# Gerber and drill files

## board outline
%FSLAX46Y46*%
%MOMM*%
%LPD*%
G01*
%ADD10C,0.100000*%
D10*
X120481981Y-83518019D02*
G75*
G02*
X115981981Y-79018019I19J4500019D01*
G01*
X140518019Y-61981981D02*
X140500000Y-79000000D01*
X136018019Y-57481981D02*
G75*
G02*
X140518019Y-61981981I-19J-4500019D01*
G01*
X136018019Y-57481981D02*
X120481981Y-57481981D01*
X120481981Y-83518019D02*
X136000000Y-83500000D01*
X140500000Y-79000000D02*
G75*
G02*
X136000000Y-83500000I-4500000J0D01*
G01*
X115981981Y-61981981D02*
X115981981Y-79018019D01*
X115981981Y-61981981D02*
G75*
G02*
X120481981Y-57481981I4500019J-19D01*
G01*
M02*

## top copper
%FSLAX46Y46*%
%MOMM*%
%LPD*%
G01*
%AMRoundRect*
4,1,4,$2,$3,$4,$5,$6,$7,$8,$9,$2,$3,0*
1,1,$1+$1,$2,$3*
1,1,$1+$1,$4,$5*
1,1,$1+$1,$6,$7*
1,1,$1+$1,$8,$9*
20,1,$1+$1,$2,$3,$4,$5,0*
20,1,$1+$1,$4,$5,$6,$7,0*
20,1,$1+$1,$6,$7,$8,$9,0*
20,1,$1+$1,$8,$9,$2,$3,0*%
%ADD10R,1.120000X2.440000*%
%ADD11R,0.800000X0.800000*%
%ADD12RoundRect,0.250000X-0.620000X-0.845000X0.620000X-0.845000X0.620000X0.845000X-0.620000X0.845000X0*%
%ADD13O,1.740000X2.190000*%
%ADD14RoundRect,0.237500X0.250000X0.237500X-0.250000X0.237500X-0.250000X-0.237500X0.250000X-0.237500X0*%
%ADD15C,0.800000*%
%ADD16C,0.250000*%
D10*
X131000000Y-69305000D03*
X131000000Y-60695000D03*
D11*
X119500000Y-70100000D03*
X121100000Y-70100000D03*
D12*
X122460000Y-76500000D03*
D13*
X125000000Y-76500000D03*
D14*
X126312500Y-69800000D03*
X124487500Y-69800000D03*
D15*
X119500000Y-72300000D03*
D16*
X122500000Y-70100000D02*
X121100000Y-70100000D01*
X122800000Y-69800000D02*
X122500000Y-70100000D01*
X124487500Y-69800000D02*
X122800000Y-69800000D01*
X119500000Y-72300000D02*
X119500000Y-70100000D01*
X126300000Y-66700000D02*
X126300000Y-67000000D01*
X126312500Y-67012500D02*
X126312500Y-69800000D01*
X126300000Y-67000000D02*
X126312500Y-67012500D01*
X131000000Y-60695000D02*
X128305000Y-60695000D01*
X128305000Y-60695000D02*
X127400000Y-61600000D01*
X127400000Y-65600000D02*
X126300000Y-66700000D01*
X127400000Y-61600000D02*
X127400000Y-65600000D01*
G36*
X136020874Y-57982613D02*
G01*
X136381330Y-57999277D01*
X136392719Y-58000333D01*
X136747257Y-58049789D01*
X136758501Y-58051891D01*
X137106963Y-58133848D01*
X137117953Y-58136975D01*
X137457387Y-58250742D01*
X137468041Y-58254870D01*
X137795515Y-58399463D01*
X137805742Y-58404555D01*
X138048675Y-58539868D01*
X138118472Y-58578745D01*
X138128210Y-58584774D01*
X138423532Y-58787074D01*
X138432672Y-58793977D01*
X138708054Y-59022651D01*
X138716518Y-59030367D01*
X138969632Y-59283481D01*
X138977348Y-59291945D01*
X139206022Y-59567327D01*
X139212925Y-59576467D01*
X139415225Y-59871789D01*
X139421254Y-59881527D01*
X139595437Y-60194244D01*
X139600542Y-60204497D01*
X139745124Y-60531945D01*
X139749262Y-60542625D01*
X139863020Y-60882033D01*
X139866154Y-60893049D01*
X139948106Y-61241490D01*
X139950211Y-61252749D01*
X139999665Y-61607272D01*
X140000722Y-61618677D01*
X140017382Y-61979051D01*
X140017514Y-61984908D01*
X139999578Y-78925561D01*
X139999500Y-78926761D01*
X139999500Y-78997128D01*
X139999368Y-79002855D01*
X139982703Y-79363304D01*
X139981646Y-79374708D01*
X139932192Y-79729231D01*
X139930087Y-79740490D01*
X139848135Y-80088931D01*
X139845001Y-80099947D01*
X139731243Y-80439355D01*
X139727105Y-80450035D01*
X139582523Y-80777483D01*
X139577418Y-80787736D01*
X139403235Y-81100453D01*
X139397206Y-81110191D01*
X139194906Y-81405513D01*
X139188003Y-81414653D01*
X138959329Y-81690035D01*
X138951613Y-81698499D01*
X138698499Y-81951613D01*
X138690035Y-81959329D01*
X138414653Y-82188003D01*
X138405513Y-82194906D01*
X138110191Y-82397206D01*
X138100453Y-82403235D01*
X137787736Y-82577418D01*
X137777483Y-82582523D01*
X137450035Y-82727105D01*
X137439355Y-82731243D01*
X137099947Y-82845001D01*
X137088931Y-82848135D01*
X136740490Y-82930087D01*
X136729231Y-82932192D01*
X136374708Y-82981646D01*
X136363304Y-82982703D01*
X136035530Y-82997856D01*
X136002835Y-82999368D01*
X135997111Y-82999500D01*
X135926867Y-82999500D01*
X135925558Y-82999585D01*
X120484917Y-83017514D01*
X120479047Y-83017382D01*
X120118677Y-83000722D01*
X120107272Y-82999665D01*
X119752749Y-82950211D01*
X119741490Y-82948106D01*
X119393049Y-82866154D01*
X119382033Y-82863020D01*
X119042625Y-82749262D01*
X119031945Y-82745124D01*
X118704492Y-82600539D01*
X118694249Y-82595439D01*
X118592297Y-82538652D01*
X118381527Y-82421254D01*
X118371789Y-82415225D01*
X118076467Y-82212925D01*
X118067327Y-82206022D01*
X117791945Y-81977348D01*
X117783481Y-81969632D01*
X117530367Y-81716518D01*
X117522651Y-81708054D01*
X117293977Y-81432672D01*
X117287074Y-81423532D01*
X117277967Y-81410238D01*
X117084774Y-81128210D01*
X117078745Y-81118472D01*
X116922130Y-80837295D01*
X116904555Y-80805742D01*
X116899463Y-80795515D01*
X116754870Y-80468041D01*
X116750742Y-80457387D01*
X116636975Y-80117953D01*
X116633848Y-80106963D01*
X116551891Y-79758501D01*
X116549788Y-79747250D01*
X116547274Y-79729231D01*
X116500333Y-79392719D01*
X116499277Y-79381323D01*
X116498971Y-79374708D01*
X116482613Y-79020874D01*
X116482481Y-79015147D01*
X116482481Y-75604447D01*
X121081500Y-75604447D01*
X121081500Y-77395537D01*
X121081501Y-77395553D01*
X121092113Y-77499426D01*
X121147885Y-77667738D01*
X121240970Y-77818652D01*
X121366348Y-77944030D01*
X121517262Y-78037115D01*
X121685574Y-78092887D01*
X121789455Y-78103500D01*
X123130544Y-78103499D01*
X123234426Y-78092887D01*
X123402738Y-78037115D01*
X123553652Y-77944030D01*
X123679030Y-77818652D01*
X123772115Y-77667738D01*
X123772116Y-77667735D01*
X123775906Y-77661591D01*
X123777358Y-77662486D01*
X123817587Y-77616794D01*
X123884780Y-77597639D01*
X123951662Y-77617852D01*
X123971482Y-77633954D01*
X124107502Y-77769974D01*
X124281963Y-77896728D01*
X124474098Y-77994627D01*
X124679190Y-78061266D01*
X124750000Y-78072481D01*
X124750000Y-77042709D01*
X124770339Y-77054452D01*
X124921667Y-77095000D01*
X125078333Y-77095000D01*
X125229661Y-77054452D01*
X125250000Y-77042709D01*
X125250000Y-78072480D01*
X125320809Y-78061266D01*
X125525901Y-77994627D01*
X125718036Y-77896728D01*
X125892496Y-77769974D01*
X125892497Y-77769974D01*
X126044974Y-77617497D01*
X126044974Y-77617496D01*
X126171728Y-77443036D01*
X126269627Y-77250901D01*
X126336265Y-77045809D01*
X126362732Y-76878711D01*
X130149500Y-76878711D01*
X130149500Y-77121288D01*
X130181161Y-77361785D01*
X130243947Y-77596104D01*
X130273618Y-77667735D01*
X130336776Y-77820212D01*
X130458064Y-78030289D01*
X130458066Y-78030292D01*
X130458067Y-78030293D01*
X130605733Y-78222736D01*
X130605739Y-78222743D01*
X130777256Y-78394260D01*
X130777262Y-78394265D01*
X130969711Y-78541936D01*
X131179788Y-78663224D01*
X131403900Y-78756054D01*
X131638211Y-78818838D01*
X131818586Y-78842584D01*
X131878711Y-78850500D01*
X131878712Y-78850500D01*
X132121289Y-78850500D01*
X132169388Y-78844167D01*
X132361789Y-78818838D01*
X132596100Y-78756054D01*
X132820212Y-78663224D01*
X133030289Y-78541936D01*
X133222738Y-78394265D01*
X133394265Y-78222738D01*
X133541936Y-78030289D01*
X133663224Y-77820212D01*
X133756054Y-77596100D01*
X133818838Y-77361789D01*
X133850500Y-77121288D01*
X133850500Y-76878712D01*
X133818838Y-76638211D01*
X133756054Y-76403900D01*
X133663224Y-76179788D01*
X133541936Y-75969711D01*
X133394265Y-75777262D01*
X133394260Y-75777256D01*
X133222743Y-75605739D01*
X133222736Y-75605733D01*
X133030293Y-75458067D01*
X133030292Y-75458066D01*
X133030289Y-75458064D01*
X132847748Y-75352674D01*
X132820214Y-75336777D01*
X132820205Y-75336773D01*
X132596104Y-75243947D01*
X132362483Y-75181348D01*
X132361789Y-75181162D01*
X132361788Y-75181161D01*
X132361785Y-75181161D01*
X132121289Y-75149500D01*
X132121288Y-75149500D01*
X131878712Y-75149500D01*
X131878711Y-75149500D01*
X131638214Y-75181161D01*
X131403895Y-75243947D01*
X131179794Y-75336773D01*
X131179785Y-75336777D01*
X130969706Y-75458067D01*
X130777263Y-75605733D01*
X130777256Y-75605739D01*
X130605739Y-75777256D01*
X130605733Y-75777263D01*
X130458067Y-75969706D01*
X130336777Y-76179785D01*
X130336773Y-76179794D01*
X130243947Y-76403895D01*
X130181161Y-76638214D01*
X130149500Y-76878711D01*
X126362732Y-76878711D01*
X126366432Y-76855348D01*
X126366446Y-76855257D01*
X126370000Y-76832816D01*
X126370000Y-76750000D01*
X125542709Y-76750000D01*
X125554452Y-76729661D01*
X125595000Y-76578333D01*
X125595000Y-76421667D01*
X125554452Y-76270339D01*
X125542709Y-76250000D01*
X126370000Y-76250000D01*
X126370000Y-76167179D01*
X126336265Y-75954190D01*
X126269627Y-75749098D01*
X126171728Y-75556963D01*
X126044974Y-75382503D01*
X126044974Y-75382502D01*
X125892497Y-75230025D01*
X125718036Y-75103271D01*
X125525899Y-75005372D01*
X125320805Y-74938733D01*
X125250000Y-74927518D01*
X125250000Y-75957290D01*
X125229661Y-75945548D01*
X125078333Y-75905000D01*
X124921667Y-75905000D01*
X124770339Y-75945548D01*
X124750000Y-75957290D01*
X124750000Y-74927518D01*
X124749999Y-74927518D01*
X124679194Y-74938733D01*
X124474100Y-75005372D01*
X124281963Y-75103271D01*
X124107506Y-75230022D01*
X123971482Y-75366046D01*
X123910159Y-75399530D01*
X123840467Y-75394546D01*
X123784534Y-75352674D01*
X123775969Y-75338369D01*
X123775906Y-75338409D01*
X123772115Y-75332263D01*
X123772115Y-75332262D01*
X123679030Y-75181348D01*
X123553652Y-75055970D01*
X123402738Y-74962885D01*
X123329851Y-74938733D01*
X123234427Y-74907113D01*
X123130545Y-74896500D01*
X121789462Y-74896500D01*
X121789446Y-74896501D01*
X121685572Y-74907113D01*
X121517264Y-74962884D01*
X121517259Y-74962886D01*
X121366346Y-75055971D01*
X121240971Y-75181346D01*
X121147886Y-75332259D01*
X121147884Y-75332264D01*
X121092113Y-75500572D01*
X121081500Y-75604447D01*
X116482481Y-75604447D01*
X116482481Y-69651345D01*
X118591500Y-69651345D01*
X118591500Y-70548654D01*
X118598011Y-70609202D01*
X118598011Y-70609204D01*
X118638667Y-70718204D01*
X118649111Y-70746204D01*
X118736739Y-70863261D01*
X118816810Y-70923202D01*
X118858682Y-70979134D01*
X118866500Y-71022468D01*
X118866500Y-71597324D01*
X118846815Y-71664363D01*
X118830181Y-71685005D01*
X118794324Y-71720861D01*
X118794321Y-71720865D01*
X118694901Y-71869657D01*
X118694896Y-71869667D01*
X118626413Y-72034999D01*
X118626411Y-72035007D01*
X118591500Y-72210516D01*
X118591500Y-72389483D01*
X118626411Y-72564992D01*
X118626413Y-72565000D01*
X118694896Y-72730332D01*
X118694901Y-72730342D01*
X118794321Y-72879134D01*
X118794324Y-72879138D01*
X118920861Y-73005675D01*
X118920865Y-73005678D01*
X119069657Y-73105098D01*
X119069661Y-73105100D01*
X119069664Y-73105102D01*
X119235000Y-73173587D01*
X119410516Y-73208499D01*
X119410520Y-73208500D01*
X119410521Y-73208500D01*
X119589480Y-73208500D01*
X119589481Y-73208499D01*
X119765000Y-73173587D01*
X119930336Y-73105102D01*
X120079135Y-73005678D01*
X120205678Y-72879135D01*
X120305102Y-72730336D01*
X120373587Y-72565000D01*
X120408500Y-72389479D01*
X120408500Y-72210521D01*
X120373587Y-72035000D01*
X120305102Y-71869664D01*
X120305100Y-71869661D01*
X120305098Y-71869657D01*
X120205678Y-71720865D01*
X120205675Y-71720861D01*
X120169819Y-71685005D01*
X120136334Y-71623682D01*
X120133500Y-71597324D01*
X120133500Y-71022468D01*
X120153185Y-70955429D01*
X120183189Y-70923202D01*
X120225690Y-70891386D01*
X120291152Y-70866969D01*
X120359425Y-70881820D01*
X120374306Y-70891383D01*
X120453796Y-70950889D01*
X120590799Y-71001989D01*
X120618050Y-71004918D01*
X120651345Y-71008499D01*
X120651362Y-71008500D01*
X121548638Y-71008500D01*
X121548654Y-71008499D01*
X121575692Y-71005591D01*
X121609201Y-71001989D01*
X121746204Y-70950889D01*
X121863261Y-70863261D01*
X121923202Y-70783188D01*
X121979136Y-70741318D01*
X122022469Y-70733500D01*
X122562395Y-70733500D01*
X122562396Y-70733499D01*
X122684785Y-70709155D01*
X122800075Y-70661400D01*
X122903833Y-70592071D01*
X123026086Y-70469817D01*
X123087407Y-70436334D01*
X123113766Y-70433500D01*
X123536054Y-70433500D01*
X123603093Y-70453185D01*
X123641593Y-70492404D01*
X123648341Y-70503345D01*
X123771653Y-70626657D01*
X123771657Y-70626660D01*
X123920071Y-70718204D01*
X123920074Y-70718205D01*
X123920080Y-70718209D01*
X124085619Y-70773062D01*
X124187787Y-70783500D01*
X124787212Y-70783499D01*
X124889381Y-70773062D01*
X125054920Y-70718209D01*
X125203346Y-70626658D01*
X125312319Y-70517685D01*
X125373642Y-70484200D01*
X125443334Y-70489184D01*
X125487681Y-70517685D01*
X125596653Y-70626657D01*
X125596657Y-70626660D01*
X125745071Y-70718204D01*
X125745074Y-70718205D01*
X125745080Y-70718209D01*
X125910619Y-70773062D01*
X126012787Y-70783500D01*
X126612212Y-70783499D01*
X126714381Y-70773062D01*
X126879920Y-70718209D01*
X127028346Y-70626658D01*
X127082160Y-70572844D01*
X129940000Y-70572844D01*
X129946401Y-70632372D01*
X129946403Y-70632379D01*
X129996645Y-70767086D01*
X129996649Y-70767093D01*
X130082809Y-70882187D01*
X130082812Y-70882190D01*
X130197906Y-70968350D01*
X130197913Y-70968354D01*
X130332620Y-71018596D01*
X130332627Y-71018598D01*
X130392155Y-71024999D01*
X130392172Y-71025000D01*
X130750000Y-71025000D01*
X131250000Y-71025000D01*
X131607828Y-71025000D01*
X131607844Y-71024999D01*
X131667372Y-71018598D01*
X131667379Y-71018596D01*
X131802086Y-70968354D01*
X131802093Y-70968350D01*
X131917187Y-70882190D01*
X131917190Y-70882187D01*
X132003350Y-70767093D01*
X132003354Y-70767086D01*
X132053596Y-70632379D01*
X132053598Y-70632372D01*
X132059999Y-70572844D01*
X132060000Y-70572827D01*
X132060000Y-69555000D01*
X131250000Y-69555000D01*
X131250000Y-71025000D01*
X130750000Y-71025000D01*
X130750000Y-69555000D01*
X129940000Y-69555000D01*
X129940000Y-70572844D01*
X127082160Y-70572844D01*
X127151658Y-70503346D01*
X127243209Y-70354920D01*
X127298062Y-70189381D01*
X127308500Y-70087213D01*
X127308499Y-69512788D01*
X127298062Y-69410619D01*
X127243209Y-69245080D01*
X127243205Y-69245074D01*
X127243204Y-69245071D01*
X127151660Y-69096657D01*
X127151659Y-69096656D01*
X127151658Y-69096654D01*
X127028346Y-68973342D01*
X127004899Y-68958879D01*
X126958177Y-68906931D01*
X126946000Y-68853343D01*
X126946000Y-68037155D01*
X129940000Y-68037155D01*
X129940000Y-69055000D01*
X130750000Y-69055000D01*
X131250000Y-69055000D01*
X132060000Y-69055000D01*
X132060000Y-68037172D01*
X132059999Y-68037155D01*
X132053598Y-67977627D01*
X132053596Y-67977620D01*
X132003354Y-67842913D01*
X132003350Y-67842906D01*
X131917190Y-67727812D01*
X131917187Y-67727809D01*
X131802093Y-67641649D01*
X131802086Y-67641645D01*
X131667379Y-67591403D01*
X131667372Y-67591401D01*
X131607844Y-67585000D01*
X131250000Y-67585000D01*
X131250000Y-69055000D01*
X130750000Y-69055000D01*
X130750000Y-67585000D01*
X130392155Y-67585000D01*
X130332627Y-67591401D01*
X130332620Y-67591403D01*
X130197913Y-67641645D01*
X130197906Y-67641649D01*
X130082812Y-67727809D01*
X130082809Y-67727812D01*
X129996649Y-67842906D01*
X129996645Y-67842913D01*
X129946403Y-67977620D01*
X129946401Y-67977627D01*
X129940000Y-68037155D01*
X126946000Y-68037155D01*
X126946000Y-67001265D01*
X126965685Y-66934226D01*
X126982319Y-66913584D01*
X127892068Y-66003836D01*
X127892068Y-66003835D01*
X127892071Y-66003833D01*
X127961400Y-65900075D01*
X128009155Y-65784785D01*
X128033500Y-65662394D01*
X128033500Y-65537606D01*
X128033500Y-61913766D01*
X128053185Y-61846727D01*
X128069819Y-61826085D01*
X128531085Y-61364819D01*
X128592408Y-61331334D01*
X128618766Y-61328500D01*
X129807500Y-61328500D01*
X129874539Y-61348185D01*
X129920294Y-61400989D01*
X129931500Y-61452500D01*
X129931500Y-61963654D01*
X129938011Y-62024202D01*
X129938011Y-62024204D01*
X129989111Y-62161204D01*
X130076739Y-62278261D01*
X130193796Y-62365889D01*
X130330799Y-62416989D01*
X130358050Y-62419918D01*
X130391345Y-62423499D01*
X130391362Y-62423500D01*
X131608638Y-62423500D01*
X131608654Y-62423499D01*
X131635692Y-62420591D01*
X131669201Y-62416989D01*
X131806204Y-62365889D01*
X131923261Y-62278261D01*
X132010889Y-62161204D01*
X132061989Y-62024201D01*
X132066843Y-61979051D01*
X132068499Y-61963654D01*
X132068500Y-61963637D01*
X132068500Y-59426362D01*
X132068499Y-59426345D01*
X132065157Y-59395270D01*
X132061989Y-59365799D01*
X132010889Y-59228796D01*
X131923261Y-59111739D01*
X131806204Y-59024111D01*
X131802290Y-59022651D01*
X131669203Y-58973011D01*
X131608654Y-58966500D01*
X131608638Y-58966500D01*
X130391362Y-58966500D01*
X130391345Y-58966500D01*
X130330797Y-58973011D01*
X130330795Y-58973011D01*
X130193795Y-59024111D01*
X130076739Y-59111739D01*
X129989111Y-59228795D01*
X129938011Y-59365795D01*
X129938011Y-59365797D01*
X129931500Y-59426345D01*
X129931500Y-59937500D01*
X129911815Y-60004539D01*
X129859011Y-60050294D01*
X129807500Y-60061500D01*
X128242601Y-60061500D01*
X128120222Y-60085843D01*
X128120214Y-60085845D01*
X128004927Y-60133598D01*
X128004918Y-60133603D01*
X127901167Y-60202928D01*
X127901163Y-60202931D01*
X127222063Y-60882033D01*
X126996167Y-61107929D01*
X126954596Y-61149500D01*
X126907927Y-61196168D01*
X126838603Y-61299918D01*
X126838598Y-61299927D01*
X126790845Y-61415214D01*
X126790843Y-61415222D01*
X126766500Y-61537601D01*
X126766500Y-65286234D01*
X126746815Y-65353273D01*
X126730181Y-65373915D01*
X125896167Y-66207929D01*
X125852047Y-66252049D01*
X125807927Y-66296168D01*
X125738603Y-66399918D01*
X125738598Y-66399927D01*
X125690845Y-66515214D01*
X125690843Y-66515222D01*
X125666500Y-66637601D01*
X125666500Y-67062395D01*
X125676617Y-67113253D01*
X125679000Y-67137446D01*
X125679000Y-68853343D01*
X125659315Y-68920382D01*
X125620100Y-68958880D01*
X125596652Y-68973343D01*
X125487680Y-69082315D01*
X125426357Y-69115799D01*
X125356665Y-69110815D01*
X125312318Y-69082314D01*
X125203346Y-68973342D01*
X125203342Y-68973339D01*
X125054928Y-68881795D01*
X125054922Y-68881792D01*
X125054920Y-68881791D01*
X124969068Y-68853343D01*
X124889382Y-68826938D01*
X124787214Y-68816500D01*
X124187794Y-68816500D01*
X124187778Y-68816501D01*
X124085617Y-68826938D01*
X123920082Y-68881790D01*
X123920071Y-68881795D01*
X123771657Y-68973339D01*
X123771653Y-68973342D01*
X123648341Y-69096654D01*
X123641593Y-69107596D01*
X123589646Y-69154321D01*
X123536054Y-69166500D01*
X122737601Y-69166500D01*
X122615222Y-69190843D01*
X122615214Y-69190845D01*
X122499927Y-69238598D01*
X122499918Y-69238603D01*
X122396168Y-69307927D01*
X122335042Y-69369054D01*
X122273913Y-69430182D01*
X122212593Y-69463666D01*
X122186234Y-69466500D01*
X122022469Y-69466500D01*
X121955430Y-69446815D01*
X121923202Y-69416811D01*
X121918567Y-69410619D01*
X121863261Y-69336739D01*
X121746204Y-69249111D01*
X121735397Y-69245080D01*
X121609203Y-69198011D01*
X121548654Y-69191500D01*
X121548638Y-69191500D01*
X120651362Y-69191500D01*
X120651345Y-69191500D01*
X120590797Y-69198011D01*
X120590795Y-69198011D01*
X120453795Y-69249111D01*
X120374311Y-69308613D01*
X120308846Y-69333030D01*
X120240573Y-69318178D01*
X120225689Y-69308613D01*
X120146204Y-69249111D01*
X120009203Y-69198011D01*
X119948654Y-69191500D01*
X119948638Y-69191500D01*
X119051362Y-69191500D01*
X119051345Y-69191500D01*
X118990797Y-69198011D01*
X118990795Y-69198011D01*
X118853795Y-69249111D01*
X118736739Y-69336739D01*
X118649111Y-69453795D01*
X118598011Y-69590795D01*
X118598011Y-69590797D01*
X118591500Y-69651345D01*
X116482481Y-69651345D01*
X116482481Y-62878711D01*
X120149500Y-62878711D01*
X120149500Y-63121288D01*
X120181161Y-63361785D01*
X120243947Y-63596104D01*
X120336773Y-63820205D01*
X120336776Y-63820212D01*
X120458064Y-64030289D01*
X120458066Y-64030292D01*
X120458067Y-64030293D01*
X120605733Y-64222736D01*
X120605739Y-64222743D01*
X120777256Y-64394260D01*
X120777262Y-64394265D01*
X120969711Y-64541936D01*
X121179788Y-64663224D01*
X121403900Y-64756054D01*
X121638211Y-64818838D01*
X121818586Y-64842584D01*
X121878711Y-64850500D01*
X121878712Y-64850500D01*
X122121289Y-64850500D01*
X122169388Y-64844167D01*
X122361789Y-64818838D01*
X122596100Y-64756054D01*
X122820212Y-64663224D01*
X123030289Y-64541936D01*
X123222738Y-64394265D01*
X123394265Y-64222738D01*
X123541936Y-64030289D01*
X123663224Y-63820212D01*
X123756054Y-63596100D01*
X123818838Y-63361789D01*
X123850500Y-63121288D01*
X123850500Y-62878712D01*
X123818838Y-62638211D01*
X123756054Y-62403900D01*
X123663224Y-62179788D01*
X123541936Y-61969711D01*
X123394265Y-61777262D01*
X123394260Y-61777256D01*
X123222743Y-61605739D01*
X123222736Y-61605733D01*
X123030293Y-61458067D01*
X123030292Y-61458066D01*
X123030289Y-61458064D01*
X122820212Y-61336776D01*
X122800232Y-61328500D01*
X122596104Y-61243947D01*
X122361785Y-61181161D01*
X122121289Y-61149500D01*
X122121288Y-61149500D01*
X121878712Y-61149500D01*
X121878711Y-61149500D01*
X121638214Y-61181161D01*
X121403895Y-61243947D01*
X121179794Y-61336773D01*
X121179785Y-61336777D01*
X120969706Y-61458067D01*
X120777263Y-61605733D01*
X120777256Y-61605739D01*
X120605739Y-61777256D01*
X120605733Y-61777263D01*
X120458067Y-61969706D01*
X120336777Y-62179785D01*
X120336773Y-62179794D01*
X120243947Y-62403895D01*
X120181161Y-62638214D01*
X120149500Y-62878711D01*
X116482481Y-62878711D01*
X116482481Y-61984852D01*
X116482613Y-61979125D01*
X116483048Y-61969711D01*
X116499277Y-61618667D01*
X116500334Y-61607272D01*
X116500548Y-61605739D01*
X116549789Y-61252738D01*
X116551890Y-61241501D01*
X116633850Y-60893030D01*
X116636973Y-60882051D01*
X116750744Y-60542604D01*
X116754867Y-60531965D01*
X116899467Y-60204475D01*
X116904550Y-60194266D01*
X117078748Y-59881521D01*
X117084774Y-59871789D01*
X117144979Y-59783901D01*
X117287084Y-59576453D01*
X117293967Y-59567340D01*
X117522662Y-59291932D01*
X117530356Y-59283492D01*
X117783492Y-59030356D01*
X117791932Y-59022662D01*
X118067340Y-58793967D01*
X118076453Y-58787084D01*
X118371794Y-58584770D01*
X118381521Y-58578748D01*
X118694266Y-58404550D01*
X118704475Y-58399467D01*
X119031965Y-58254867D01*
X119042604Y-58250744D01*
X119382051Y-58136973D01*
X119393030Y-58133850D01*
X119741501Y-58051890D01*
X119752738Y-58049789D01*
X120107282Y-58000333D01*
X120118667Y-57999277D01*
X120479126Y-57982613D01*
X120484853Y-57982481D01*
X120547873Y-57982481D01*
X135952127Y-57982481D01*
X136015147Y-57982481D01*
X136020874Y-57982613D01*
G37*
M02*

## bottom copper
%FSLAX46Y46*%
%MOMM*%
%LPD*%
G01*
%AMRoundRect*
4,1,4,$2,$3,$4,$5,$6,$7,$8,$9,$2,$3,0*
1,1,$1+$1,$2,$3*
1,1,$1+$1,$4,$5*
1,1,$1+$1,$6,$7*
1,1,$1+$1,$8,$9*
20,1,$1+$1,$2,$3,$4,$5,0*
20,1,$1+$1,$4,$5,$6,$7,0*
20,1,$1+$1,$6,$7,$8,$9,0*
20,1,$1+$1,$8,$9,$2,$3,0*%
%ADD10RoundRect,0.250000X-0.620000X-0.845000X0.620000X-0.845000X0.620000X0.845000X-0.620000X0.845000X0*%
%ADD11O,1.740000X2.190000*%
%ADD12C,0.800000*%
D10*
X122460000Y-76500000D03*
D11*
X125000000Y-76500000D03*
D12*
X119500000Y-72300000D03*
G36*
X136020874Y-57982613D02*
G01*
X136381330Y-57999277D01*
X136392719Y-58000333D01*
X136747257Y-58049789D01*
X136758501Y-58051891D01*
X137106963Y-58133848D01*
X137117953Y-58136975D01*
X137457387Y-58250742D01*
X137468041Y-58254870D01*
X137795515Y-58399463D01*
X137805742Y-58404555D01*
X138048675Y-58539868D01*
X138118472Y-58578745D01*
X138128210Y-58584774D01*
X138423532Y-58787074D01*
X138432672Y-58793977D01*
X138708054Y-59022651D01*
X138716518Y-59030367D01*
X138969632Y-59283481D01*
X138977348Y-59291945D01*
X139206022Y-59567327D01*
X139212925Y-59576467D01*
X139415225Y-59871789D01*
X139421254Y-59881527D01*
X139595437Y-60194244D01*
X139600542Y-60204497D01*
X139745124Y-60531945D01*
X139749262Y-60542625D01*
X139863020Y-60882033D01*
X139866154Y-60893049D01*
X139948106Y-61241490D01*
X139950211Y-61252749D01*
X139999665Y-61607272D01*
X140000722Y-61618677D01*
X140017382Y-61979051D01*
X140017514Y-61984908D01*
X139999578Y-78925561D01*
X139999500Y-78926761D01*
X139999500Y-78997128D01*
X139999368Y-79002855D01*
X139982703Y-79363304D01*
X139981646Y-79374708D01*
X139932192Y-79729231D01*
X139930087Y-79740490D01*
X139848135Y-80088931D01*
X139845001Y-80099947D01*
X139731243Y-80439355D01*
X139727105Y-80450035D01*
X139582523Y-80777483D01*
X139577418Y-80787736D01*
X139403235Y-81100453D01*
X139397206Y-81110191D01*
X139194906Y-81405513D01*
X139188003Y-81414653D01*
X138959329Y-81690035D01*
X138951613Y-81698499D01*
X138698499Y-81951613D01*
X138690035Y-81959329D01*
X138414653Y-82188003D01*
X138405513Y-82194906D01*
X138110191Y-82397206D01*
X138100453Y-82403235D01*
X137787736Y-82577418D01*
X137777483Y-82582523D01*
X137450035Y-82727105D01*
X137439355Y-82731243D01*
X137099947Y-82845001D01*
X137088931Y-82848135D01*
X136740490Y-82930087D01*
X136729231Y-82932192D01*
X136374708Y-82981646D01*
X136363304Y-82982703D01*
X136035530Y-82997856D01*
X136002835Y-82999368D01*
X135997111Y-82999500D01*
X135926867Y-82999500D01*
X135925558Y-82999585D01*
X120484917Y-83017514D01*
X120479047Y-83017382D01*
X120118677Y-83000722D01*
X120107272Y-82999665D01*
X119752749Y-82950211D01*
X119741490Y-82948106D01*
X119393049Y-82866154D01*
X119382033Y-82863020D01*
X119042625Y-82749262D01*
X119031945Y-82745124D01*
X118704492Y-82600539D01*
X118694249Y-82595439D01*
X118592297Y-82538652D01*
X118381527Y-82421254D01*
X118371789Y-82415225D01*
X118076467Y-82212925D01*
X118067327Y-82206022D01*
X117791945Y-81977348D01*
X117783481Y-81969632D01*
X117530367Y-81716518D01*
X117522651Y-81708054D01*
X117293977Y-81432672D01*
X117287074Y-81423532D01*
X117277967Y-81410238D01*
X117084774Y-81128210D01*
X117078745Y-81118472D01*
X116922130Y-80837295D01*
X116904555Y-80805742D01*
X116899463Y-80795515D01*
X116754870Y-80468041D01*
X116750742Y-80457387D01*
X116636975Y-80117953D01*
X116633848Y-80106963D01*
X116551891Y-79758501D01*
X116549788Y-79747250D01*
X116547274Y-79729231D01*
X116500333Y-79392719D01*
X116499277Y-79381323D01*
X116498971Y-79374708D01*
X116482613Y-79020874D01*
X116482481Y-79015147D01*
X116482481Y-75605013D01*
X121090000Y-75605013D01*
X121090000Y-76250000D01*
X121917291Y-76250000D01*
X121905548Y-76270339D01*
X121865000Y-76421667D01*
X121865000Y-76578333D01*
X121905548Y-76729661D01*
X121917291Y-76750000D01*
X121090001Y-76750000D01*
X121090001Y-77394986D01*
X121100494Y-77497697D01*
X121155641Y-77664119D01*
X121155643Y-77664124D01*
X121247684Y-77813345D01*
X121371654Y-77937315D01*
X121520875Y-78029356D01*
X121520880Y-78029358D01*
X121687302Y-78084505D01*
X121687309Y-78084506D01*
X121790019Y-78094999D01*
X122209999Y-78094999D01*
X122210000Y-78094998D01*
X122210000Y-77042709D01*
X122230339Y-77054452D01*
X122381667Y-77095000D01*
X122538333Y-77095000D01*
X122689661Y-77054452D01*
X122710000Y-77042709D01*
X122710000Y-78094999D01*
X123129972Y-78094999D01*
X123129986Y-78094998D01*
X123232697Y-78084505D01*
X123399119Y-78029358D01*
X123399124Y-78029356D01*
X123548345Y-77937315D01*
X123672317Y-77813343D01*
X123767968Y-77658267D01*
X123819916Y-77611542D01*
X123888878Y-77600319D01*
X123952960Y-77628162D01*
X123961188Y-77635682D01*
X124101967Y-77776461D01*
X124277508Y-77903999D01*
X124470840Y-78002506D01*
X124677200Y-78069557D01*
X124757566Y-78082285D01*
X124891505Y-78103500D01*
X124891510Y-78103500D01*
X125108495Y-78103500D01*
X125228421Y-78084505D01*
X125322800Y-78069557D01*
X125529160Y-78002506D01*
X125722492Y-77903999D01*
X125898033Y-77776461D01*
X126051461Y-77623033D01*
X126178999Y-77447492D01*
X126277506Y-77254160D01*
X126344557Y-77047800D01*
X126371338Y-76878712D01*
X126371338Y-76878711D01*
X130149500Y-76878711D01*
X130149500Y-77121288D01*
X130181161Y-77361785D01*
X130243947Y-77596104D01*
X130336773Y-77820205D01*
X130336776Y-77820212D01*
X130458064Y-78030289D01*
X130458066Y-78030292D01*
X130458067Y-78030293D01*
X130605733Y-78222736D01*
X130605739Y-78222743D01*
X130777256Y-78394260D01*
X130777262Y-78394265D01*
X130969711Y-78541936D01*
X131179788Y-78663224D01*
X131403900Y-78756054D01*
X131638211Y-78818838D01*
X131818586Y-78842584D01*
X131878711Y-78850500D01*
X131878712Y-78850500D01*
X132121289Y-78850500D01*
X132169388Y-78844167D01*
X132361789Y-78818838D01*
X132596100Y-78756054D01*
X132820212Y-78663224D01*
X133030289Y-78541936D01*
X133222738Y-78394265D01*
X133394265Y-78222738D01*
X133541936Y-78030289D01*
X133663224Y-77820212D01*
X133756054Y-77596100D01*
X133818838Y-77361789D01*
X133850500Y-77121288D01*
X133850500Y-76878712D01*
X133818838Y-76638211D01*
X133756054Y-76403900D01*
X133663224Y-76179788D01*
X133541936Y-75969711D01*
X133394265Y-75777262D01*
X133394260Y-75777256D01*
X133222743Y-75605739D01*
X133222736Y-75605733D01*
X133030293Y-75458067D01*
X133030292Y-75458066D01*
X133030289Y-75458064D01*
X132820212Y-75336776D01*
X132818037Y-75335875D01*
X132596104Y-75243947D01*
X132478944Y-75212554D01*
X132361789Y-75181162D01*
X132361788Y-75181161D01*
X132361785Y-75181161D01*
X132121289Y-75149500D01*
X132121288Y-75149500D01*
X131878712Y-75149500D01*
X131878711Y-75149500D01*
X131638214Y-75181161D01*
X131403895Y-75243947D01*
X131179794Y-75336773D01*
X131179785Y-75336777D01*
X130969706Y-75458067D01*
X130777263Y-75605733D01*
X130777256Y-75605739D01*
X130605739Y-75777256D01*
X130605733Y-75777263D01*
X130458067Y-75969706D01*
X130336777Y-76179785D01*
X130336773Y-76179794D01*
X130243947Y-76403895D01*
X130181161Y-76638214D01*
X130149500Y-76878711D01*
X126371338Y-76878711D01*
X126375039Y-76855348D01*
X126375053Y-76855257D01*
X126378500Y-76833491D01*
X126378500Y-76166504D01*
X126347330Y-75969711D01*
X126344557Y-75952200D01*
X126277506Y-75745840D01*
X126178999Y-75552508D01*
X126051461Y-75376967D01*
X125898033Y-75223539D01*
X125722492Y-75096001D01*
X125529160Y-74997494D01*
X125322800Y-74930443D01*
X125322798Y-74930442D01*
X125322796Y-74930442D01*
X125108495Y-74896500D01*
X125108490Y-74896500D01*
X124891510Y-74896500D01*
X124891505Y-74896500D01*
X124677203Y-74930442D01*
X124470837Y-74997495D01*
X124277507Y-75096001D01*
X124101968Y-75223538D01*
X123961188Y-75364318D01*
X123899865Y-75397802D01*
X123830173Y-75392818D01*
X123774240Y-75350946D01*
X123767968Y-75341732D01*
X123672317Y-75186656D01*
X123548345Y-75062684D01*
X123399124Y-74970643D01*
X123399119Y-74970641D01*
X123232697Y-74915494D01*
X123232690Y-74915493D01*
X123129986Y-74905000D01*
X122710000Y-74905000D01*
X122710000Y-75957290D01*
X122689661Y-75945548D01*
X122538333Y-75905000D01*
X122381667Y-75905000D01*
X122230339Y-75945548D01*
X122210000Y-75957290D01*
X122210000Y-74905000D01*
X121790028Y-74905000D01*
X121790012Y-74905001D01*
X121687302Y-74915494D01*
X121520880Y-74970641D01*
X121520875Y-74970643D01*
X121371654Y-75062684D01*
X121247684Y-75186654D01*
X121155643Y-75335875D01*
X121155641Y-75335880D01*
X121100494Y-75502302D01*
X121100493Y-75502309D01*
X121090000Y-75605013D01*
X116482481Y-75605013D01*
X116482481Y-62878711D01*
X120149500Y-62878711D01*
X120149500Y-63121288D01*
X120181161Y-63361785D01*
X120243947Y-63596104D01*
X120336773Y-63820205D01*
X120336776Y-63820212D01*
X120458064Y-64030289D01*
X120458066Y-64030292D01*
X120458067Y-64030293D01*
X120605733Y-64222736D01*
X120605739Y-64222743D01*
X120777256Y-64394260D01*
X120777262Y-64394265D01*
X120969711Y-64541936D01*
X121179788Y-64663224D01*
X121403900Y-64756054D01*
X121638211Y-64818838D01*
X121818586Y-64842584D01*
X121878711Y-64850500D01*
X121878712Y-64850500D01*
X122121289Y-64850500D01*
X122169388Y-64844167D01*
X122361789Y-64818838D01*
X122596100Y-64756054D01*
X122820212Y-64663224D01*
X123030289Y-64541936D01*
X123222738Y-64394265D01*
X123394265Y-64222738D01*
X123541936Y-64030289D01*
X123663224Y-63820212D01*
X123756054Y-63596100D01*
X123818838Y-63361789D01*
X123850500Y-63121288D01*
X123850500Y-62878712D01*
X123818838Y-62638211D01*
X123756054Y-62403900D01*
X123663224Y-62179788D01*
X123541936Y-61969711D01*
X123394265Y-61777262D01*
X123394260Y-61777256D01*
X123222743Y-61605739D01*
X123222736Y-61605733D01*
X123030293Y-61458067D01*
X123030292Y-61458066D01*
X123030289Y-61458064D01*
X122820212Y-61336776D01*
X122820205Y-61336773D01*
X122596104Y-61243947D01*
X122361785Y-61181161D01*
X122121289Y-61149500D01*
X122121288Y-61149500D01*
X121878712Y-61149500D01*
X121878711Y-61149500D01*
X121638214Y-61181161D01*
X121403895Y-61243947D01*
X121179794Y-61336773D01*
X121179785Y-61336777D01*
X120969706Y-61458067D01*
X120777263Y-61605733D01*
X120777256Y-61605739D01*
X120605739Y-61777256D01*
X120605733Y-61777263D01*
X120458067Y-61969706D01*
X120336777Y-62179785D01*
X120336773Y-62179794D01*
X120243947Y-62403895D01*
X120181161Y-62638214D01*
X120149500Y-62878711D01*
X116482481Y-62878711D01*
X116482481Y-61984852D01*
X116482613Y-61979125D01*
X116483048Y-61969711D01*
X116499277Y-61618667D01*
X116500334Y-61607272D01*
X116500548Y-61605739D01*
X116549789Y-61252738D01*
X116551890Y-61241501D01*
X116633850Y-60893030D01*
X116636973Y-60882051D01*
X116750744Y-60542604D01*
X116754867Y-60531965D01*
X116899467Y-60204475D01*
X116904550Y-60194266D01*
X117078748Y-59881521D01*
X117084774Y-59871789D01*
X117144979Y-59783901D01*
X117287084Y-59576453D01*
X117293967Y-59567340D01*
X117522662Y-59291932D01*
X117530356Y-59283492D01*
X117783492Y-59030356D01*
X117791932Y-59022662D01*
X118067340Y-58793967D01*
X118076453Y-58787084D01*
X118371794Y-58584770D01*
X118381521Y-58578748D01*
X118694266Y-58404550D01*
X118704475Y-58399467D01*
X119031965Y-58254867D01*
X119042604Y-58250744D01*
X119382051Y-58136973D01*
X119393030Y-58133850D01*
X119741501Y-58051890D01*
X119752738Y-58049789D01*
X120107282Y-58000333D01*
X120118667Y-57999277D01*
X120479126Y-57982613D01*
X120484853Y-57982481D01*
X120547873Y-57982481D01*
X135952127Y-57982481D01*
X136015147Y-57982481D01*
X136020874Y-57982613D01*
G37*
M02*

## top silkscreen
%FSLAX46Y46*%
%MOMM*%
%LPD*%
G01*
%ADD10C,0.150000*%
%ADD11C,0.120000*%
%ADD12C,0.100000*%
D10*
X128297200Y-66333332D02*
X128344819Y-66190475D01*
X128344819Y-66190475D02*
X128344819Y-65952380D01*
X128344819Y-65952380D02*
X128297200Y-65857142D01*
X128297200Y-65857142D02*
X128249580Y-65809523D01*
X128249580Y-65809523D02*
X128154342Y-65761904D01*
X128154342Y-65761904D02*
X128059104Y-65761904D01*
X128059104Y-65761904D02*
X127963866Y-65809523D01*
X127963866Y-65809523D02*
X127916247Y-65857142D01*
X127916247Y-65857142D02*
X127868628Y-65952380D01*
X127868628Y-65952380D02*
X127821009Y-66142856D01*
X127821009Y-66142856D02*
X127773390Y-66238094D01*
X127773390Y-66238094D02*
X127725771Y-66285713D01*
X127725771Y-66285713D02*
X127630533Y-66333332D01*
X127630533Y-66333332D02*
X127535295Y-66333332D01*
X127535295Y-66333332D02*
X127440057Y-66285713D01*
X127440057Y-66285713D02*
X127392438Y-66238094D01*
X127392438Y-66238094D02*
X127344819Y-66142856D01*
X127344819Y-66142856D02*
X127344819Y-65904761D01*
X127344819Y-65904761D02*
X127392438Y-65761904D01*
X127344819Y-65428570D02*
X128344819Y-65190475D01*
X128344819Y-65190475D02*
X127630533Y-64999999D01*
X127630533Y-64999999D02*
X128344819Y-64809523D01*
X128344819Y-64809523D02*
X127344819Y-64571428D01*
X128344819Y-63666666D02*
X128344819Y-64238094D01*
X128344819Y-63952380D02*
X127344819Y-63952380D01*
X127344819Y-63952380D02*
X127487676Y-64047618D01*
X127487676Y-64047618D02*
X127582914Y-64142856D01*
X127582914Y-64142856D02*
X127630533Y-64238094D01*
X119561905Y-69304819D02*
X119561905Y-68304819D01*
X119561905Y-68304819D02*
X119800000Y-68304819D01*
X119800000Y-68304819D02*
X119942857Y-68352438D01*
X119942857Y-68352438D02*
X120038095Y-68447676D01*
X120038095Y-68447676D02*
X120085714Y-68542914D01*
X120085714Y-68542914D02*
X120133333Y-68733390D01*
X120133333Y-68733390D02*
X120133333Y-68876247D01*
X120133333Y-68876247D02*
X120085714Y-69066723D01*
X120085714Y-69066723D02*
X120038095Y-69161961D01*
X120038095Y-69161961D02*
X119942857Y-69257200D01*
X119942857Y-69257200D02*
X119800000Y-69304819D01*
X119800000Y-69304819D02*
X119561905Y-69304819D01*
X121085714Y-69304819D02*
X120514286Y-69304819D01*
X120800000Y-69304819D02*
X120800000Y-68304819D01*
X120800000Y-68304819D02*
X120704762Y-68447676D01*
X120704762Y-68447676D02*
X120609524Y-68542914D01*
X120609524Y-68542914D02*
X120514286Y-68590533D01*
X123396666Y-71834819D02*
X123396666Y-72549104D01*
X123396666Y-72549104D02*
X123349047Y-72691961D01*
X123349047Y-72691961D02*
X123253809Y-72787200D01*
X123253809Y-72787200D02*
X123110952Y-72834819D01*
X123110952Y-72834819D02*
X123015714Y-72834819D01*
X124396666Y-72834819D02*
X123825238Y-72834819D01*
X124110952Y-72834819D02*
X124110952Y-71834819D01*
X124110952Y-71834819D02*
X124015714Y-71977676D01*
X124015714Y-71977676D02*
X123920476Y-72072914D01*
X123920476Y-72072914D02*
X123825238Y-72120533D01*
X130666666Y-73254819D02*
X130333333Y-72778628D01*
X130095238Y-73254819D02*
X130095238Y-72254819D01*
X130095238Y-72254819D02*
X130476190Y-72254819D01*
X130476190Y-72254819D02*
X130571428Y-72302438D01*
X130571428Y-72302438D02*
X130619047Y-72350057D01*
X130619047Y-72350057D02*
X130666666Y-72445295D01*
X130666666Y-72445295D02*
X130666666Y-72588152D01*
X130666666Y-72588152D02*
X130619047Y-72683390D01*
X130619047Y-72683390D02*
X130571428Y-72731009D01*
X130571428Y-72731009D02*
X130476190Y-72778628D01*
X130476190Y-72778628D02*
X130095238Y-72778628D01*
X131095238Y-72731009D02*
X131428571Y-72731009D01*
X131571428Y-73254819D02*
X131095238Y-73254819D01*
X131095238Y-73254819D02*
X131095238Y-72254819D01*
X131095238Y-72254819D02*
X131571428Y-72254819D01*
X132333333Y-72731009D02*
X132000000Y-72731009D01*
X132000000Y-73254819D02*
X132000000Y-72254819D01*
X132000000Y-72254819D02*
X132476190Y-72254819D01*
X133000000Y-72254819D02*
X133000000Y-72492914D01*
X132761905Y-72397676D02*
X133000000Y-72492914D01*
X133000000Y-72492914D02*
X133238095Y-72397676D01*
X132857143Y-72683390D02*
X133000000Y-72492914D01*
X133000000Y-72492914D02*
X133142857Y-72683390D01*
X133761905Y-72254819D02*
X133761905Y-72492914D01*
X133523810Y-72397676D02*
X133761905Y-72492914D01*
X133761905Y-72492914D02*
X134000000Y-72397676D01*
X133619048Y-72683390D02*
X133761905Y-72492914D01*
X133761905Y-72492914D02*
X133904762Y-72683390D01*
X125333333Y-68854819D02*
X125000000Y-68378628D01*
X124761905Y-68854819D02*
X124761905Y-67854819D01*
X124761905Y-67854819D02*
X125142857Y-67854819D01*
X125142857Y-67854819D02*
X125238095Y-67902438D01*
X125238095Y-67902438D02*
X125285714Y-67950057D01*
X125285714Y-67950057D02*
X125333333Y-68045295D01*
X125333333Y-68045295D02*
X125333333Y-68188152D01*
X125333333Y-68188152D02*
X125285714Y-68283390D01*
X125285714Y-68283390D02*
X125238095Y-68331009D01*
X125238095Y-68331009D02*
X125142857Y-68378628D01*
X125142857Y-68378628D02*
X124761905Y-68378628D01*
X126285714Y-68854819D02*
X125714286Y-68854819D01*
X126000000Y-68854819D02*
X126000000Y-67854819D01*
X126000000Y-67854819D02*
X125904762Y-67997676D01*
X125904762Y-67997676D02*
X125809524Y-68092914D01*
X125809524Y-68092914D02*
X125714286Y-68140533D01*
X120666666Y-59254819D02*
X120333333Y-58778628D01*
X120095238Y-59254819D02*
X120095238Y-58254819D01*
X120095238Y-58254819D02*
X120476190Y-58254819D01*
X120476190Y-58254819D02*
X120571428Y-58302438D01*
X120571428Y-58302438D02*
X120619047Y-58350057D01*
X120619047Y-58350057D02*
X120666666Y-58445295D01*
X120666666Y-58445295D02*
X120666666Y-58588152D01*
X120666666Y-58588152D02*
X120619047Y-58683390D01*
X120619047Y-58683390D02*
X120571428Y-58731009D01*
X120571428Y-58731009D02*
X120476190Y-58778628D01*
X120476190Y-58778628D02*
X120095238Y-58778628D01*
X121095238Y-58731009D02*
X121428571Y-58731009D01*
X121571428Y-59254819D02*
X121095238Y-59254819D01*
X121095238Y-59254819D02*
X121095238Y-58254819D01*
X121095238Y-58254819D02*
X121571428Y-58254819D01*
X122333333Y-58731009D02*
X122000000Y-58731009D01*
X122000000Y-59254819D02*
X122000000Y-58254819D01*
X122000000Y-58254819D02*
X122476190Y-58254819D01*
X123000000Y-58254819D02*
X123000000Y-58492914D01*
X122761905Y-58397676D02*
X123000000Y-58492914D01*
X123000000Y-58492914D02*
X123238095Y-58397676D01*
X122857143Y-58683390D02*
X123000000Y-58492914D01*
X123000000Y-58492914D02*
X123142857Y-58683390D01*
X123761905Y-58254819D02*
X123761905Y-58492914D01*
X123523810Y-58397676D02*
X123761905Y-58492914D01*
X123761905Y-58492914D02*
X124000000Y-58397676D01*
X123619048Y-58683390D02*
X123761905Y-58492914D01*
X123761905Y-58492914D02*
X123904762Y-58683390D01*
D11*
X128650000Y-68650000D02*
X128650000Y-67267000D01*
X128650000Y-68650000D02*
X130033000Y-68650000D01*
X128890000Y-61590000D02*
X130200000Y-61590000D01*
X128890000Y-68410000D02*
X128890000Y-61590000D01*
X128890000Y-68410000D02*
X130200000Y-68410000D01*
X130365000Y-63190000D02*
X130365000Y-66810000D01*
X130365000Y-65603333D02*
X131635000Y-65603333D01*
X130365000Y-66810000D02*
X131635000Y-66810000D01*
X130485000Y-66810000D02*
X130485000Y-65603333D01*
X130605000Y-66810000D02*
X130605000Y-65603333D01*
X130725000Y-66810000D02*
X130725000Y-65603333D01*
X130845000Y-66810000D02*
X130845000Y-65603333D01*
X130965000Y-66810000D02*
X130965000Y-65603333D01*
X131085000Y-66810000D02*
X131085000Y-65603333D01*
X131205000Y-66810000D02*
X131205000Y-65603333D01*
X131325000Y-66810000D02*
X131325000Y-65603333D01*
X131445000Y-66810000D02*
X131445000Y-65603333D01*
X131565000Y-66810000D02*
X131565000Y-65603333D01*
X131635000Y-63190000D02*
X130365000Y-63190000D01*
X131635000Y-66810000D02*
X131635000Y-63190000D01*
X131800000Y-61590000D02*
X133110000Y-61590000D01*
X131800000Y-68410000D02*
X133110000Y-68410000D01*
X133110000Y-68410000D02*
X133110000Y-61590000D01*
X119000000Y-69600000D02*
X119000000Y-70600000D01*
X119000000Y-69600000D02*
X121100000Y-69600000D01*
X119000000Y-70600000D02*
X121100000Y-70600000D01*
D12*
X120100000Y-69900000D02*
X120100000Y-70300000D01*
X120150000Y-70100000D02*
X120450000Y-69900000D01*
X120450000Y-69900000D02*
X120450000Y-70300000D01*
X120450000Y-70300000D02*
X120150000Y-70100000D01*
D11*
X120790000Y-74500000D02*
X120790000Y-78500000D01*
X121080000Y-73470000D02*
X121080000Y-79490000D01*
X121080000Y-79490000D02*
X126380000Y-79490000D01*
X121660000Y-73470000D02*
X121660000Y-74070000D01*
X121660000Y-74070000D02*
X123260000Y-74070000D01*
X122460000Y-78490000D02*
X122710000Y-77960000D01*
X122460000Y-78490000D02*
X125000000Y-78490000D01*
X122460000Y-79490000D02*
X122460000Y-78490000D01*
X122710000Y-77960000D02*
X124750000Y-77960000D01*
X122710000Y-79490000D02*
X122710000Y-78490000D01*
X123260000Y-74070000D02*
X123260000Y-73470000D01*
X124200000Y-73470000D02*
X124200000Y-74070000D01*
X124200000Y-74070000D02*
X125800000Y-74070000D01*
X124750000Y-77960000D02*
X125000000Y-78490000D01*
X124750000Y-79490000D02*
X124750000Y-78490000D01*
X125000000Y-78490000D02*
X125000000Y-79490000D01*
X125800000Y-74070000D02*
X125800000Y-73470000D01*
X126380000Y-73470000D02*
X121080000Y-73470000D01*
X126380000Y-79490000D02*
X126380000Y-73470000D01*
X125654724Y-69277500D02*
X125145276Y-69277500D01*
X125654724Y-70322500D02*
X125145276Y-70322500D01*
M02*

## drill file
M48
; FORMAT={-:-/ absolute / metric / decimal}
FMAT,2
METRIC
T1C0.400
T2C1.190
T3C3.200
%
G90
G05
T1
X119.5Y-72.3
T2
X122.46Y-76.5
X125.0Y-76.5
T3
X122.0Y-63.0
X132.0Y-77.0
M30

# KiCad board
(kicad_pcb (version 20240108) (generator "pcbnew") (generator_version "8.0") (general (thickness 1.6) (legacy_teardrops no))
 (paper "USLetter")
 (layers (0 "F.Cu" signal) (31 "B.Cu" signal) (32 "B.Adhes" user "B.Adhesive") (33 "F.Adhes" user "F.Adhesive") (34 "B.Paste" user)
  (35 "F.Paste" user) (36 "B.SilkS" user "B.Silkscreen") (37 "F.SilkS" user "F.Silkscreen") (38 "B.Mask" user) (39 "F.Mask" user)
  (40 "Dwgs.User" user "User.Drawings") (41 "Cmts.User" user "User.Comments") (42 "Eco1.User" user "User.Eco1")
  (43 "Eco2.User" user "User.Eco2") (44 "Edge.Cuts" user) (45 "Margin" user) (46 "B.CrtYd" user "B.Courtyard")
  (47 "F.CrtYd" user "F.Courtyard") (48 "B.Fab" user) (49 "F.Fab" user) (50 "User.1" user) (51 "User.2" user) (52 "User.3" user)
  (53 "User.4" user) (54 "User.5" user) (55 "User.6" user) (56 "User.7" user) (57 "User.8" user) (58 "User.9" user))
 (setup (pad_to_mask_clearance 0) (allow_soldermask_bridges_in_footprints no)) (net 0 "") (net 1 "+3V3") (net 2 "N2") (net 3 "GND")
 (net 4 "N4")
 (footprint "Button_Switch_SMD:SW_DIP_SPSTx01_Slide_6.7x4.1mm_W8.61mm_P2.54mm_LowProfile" (layer "F.Cu") (at 131 65 90)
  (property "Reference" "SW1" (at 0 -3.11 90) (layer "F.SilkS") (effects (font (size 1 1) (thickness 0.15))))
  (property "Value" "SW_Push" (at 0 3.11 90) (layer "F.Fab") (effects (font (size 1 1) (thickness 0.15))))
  (fp_line (start -3.65 -2.35) (end -2.267 -2.35) (stroke (width 0.12) (type solid)) (layer "F.SilkS"))
  (fp_line (start -3.65 -2.35) (end -3.65 -0.967) (stroke (width 0.12) (type solid)) (layer "F.SilkS"))
  (fp_line (start 3.41 -2.11) (end 3.41 -0.8) (stroke (width 0.12) (type solid)) (layer "F.SilkS"))
  (fp_line (start -3.41 -2.11) (end 3.41 -2.11) (stroke (width 0.12) (type solid)) (layer "F.SilkS"))
  (fp_line (start -3.41 -2.11) (end -3.41 -0.8) (stroke (width 0.12) (type solid)) (layer "F.SilkS"))
  (fp_line (start 1.81 -0.635) (end -1.81 -0.635) (stroke (width 0.12) (type solid)) (layer "F.SilkS"))
  (fp_line (start -0.603333 -0.635) (end -0.603333 0.635) (stroke (width 0.12) (type solid)) (layer "F.SilkS"))
  (fp_line (start -1.81 -0.635) (end -1.81 0.635) (stroke (width 0.12) (type solid)) (layer "F.SilkS"))
  (fp_line (start -1.81 -0.515) (end -0.603333 -0.515) (stroke (width 0.12) (type solid)) (layer "F.SilkS"))
  (fp_line (start -1.81 -0.395) (end -0.603333 -0.395) (stroke (width 0.12) (type solid)) (layer "F.SilkS"))
  (fp_line (start -1.81 -0.275) (end -0.603333 -0.275) (stroke (width 0.12) (type solid)) (layer "F.SilkS"))
  (fp_line (start -1.81 -0.155) (end -0.603333 -0.155) (stroke (width 0.12) (type solid)) (layer "F.SilkS"))
  (fp_line (start -1.81 -0.035) (end -0.603333 -0.035) (stroke (width 0.12) (type solid)) (layer "F.SilkS"))
  (fp_line (start -1.81 0.085) (end -0.603333 0.085) (stroke (width 0.12) (type solid)) (layer "F.SilkS"))
  (fp_line (start -1.81 0.205) (end -0.603333 0.205) (stroke (width 0.12) (type solid)) (layer "F.SilkS"))
  (fp_line (start -1.81 0.325) (end -0.603333 0.325) (stroke (width 0.12) (type solid)) (layer "F.SilkS"))
  (fp_line (start -1.81 0.445) (end -0.603333 0.445) (stroke (width 0.12) (type solid)) (layer "F.SilkS"))
  (fp_line (start -1.81 0.565) (end -0.603333 0.565) (stroke (width 0.12) (type solid)) (layer "F.SilkS"))
  (fp_line (start 1.81 0.635) (end 1.81 -0.635) (stroke (width 0.12) (type solid)) (layer "F.SilkS"))
  (fp_line (start -1.81 0.635) (end 1.81 0.635) (stroke (width 0.12) (type solid)) (layer "F.SilkS"))
  (fp_line (start 3.41 0.8) (end 3.41 2.11) (stroke (width 0.12) (type solid)) (layer "F.SilkS"))
  (fp_line (start -3.41 0.8) (end -3.41 2.11) (stroke (width 0.12) (type solid)) (layer "F.SilkS"))
  (fp_line (start -3.41 2.11) (end 3.41 2.11) (stroke (width 0.12) (type solid)) (layer "F.SilkS"))
  (pad "1" smd rect (at -4.305 0 90) (size 2.44 1.12) (layers "F.Cu" "F.Paste" "F.Mask") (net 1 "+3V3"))
  (pad "2" smd rect (at 4.305 0 90) (size 2.44 1.12) (layers "F.Cu" "F.Paste" "F.Mask") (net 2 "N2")))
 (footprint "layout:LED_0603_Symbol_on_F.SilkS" (layer "F.Cu") (at 120.3 70.1)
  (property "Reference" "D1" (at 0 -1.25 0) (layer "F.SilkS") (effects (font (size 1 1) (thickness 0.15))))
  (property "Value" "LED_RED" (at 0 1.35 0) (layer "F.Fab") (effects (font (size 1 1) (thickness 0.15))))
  (fp_line (start -1.3 -0.5) (end -1.3 0.5) (stroke (width 0.12) (type solid)) (layer "F.SilkS"))
  (fp_line (start -1.3 -0.5) (end 0.8 -0.5) (stroke (width 0.12) (type solid)) (layer "F.SilkS"))
  (fp_line (start -1.3 0.5) (end 0.8 0.5) (stroke (width 0.12) (type solid)) (layer "F.SilkS"))
  (fp_line (start -0.2 -0.2) (end -0.2 0.2) (stroke (width 0.1) (type solid)) (layer "F.SilkS"))
  (fp_line (start -0.15 0) (end 0.15 -0.2) (stroke (width 0.1) (type solid)) (layer "F.SilkS"))
  (fp_line (start 0.15 -0.2) (end 0.15 0.2) (stroke (width 0.1) (type solid)) (layer "F.SilkS"))
  (fp_line (start 0.15 0.2) (end -0.15 0) (stroke (width 0.1) (type solid)) (layer "F.SilkS"))
  (pad "1" smd rect (at -0.8 0 180) (size 0.8 0.8) (layers "F.Cu" "F.Paste" "F.Mask") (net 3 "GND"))
  (pad "2" smd rect (at 0.8 0 180) (size 0.8 0.8) (layers "F.Cu" "F.Paste" "F.Mask") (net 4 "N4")))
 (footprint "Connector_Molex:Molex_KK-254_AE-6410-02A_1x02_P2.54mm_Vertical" (layer "F.Cu") (at 122.46 76.5)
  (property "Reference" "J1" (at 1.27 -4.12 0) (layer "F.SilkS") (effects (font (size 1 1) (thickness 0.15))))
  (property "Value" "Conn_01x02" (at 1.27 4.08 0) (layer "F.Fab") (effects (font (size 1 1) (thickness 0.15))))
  (fp_line (start -1.67 -2) (end -1.67 2) (stroke (width 0.12) (type solid)) (layer "F.SilkS"))
  (fp_line (start -1.38 -3.03) (end -1.38 2.99) (stroke (width 0.12) (type solid)) (layer "F.SilkS"))
  (fp_line (start -1.38 2.99) (end 3.92 2.99) (stroke (width 0.12) (type solid)) (layer "F.SilkS"))
  (fp_line (start -0.8 -3.03) (end -0.8 -2.43) (stroke (width 0.12) (type solid)) (layer "F.SilkS"))
  (fp_line (start -0.8 -2.43) (end 0.8 -2.43) (stroke (width 0.12) (type solid)) (layer "F.SilkS"))
  (fp_line (start 0 1.99) (end 0.25 1.46) (stroke (width 0.12) (type solid)) (layer "F.SilkS"))
  (fp_line (start 0 1.99) (end 2.54 1.99) (stroke (width 0.12) (type solid)) (layer "F.SilkS"))
  (fp_line (start 0 2.99) (end 0 1.99) (stroke (width 0.12) (type solid)) (layer "F.SilkS"))
  (fp_line (start 0.25 1.46) (end 2.29 1.46) (stroke (width 0.12) (type solid)) (layer "F.SilkS"))
  (fp_line (start 0.25 2.99) (end 0.25 1.99) (stroke (width 0.12) (type solid)) (layer "F.SilkS"))
  (fp_line (start 0.8 -2.43) (end 0.8 -3.03) (stroke (width 0.12) (type solid)) (layer "F.SilkS"))
  (fp_line (start 1.74 -3.03) (end 1.74 -2.43) (stroke (width 0.12) (type solid)) (layer "F.SilkS"))
  (fp_line (start 1.74 -2.43) (end 3.34 -2.43) (stroke (width 0.12) (type solid)) (layer "F.SilkS"))
  (fp_line (start 2.29 1.46) (end 2.54 1.99) (stroke (width 0.12) (type solid)) (layer "F.SilkS"))
  (fp_line (start 2.29 2.99) (end 2.29 1.99) (stroke (width 0.12) (type solid)) (layer "F.SilkS"))
  (fp_line (start 2.54 1.99) (end 2.54 2.99) (stroke (width 0.12) (type solid)) (layer "F.SilkS"))
  (fp_line (start 3.34 -2.43) (end 3.34 -3.03) (stroke (width 0.12) (type solid)) (layer "F.SilkS"))
  (fp_line (start 3.92 -3.03) (end -1.38 -3.03) (stroke (width 0.12) (type solid)) (layer "F.SilkS"))
  (fp_line (start 3.92 2.99) (end 3.92 -3.03) (stroke (width 0.12) (type solid)) (layer "F.SilkS"))
  (pad "1" thru_hole roundrect (at 0 0) (size 1.74 2.19) (drill 1.19) (layers "*.Cu" "*.Mask") (remove_unused_layers no)
   (roundrect_rratio 0.143678) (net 3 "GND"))
  (pad "2" thru_hole oval (at 2.54 0) (size 1.74 2.19) (drill 1.19) (layers "*.Cu" "*.Mask") (remove_unused_layers no) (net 1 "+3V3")))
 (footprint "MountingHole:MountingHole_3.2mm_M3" (layer "F.Cu") (at 132 77)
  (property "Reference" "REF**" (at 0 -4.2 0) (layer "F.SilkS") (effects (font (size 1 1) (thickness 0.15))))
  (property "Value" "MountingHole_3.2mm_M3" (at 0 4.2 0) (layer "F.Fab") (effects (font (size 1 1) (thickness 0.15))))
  (pad "" np_thru_hole circle (at 0 0) (size 3.2 3.2) (drill 3.2) (layers "*.Cu" "*.Mask")))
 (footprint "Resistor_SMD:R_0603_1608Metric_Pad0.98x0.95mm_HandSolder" (layer "F.Cu") (at 125.4 69.8 180)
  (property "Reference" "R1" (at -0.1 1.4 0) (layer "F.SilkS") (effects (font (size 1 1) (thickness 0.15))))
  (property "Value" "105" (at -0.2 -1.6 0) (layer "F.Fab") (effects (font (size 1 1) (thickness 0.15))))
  (fp_line (start -0.254724 0.5225) (end 0.254724 0.5225) (stroke (width 0.12) (type solid)) (layer "F.SilkS"))
  (fp_line (start -0.254724 -0.5225) (end 0.254724 -0.5225) (stroke (width 0.12) (type solid)) (layer "F.SilkS"))
  (pad "1" smd roundrect (at -0.9125 0 180) (size 0.975 0.95) (layers "F.Cu" "F.Paste" "F.Mask") (roundrect_rratio 0.25) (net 2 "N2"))
  (pad "2" smd roundrect (at 0.9125 0 180) (size 0.975 0.95) (layers "F.Cu" "F.Paste" "F.Mask") (roundrect_rratio 0.25) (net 4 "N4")))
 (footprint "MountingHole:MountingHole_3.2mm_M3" (layer "F.Cu") (at 122 63)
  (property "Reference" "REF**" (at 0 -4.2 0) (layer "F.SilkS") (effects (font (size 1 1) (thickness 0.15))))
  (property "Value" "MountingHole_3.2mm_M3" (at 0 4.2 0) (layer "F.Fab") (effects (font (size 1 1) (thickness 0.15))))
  (pad "" np_thru_hole circle (at 0 0) (size 3.2 3.2) (drill 3.2) (layers "*.Cu" "*.Mask")))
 (gr_arc (start 120.481981 83.518019) (mid 117.3 82.2) (end 115.981981 79.018019) (stroke (width 0.1) (type default)) (layer "Edge.Cuts"))
 (gr_line (start 140.518019 61.981981) (end 140.5 79) (stroke (width 0.1) (type default)) (layer "Edge.Cuts"))
 (gr_arc (start 136.018019 57.481981) (mid 139.2 58.8) (end 140.518019 61.981981) (stroke (width 0.1) (type default)) (layer "Edge.Cuts"))
 (gr_line (start 136.018019 57.481981) (end 120.481981 57.481981) (stroke (width 0.1) (type default)) (layer "Edge.Cuts"))
 (gr_line (start 120.481981 83.518019) (end 136 83.5) (stroke (width 0.1) (type default)) (layer "Edge.Cuts"))
 (gr_arc (start 140.5 79) (mid 139.181981 82.181981) (end 136 83.5) (stroke (width 0.1) (type default)) (layer "Edge.Cuts"))
 (gr_line (start 115.981981 61.981981) (end 115.981981 79.018019) (stroke (width 0.1) (type default)) (layer "Edge.Cuts"))
 (gr_arc (start 115.981981 61.981981) (mid 117.3 58.8) (end 120.481981 57.481981) (stroke (width 0.1) (type default)) (layer "Edge.Cuts"))
 (segment (start 122.5 70.1) (end 121.1 70.1) (width 0.25) (layer "F.Cu") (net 4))
 (segment (start 122.8 69.8) (end 122.5 70.1) (width 0.25) (layer "F.Cu") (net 4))
 (segment (start 124.4875 69.8) (end 122.8 69.8) (width 0.25) (layer "F.Cu") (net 4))
 (segment (start 119.5 72.3) (end 119.5 70.1) (width 0.25) (layer "F.Cu") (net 3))
 (via (at 119.5 72.3) (size 0.8) (drill 0.4) (layers "F.Cu" "B.Cu") (free yes) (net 3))
 (segment (start 126.3 66.7) (end 126.3 67) (width 0.25) (layer "F.Cu") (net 2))
 (segment (start 126.3125 67.0125) (end 126.3125 69.8) (width 0.25) (layer "F.Cu") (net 2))
 (segment (start 126.3 67) (end 126.3125 67.0125) (width 0.25) (layer "F.Cu") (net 2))
 (segment (start 131 60.695) (end 128.305 60.695) (width 0.25) (layer "F.Cu") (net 2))
 (segment (start 128.305 60.695) (end 127.4 61.6) (width 0.25) (layer "F.Cu") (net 2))
 (segment (start 127.4 65.6) (end 126.3 66.7) (width 0.25) (layer "F.Cu") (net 2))
 (segment (start 127.4 61.6) (end 127.4 65.6) (width 0.25) (layer "F.Cu") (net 2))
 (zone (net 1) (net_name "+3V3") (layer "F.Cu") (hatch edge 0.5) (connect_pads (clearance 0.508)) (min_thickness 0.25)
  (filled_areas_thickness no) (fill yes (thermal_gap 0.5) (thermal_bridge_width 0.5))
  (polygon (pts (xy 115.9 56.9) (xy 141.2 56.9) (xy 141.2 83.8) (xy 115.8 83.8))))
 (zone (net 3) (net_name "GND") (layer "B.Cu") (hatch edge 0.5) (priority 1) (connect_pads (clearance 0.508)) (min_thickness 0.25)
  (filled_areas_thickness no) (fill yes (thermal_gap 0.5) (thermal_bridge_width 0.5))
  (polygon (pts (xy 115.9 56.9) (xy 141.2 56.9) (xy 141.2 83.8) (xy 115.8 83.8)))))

